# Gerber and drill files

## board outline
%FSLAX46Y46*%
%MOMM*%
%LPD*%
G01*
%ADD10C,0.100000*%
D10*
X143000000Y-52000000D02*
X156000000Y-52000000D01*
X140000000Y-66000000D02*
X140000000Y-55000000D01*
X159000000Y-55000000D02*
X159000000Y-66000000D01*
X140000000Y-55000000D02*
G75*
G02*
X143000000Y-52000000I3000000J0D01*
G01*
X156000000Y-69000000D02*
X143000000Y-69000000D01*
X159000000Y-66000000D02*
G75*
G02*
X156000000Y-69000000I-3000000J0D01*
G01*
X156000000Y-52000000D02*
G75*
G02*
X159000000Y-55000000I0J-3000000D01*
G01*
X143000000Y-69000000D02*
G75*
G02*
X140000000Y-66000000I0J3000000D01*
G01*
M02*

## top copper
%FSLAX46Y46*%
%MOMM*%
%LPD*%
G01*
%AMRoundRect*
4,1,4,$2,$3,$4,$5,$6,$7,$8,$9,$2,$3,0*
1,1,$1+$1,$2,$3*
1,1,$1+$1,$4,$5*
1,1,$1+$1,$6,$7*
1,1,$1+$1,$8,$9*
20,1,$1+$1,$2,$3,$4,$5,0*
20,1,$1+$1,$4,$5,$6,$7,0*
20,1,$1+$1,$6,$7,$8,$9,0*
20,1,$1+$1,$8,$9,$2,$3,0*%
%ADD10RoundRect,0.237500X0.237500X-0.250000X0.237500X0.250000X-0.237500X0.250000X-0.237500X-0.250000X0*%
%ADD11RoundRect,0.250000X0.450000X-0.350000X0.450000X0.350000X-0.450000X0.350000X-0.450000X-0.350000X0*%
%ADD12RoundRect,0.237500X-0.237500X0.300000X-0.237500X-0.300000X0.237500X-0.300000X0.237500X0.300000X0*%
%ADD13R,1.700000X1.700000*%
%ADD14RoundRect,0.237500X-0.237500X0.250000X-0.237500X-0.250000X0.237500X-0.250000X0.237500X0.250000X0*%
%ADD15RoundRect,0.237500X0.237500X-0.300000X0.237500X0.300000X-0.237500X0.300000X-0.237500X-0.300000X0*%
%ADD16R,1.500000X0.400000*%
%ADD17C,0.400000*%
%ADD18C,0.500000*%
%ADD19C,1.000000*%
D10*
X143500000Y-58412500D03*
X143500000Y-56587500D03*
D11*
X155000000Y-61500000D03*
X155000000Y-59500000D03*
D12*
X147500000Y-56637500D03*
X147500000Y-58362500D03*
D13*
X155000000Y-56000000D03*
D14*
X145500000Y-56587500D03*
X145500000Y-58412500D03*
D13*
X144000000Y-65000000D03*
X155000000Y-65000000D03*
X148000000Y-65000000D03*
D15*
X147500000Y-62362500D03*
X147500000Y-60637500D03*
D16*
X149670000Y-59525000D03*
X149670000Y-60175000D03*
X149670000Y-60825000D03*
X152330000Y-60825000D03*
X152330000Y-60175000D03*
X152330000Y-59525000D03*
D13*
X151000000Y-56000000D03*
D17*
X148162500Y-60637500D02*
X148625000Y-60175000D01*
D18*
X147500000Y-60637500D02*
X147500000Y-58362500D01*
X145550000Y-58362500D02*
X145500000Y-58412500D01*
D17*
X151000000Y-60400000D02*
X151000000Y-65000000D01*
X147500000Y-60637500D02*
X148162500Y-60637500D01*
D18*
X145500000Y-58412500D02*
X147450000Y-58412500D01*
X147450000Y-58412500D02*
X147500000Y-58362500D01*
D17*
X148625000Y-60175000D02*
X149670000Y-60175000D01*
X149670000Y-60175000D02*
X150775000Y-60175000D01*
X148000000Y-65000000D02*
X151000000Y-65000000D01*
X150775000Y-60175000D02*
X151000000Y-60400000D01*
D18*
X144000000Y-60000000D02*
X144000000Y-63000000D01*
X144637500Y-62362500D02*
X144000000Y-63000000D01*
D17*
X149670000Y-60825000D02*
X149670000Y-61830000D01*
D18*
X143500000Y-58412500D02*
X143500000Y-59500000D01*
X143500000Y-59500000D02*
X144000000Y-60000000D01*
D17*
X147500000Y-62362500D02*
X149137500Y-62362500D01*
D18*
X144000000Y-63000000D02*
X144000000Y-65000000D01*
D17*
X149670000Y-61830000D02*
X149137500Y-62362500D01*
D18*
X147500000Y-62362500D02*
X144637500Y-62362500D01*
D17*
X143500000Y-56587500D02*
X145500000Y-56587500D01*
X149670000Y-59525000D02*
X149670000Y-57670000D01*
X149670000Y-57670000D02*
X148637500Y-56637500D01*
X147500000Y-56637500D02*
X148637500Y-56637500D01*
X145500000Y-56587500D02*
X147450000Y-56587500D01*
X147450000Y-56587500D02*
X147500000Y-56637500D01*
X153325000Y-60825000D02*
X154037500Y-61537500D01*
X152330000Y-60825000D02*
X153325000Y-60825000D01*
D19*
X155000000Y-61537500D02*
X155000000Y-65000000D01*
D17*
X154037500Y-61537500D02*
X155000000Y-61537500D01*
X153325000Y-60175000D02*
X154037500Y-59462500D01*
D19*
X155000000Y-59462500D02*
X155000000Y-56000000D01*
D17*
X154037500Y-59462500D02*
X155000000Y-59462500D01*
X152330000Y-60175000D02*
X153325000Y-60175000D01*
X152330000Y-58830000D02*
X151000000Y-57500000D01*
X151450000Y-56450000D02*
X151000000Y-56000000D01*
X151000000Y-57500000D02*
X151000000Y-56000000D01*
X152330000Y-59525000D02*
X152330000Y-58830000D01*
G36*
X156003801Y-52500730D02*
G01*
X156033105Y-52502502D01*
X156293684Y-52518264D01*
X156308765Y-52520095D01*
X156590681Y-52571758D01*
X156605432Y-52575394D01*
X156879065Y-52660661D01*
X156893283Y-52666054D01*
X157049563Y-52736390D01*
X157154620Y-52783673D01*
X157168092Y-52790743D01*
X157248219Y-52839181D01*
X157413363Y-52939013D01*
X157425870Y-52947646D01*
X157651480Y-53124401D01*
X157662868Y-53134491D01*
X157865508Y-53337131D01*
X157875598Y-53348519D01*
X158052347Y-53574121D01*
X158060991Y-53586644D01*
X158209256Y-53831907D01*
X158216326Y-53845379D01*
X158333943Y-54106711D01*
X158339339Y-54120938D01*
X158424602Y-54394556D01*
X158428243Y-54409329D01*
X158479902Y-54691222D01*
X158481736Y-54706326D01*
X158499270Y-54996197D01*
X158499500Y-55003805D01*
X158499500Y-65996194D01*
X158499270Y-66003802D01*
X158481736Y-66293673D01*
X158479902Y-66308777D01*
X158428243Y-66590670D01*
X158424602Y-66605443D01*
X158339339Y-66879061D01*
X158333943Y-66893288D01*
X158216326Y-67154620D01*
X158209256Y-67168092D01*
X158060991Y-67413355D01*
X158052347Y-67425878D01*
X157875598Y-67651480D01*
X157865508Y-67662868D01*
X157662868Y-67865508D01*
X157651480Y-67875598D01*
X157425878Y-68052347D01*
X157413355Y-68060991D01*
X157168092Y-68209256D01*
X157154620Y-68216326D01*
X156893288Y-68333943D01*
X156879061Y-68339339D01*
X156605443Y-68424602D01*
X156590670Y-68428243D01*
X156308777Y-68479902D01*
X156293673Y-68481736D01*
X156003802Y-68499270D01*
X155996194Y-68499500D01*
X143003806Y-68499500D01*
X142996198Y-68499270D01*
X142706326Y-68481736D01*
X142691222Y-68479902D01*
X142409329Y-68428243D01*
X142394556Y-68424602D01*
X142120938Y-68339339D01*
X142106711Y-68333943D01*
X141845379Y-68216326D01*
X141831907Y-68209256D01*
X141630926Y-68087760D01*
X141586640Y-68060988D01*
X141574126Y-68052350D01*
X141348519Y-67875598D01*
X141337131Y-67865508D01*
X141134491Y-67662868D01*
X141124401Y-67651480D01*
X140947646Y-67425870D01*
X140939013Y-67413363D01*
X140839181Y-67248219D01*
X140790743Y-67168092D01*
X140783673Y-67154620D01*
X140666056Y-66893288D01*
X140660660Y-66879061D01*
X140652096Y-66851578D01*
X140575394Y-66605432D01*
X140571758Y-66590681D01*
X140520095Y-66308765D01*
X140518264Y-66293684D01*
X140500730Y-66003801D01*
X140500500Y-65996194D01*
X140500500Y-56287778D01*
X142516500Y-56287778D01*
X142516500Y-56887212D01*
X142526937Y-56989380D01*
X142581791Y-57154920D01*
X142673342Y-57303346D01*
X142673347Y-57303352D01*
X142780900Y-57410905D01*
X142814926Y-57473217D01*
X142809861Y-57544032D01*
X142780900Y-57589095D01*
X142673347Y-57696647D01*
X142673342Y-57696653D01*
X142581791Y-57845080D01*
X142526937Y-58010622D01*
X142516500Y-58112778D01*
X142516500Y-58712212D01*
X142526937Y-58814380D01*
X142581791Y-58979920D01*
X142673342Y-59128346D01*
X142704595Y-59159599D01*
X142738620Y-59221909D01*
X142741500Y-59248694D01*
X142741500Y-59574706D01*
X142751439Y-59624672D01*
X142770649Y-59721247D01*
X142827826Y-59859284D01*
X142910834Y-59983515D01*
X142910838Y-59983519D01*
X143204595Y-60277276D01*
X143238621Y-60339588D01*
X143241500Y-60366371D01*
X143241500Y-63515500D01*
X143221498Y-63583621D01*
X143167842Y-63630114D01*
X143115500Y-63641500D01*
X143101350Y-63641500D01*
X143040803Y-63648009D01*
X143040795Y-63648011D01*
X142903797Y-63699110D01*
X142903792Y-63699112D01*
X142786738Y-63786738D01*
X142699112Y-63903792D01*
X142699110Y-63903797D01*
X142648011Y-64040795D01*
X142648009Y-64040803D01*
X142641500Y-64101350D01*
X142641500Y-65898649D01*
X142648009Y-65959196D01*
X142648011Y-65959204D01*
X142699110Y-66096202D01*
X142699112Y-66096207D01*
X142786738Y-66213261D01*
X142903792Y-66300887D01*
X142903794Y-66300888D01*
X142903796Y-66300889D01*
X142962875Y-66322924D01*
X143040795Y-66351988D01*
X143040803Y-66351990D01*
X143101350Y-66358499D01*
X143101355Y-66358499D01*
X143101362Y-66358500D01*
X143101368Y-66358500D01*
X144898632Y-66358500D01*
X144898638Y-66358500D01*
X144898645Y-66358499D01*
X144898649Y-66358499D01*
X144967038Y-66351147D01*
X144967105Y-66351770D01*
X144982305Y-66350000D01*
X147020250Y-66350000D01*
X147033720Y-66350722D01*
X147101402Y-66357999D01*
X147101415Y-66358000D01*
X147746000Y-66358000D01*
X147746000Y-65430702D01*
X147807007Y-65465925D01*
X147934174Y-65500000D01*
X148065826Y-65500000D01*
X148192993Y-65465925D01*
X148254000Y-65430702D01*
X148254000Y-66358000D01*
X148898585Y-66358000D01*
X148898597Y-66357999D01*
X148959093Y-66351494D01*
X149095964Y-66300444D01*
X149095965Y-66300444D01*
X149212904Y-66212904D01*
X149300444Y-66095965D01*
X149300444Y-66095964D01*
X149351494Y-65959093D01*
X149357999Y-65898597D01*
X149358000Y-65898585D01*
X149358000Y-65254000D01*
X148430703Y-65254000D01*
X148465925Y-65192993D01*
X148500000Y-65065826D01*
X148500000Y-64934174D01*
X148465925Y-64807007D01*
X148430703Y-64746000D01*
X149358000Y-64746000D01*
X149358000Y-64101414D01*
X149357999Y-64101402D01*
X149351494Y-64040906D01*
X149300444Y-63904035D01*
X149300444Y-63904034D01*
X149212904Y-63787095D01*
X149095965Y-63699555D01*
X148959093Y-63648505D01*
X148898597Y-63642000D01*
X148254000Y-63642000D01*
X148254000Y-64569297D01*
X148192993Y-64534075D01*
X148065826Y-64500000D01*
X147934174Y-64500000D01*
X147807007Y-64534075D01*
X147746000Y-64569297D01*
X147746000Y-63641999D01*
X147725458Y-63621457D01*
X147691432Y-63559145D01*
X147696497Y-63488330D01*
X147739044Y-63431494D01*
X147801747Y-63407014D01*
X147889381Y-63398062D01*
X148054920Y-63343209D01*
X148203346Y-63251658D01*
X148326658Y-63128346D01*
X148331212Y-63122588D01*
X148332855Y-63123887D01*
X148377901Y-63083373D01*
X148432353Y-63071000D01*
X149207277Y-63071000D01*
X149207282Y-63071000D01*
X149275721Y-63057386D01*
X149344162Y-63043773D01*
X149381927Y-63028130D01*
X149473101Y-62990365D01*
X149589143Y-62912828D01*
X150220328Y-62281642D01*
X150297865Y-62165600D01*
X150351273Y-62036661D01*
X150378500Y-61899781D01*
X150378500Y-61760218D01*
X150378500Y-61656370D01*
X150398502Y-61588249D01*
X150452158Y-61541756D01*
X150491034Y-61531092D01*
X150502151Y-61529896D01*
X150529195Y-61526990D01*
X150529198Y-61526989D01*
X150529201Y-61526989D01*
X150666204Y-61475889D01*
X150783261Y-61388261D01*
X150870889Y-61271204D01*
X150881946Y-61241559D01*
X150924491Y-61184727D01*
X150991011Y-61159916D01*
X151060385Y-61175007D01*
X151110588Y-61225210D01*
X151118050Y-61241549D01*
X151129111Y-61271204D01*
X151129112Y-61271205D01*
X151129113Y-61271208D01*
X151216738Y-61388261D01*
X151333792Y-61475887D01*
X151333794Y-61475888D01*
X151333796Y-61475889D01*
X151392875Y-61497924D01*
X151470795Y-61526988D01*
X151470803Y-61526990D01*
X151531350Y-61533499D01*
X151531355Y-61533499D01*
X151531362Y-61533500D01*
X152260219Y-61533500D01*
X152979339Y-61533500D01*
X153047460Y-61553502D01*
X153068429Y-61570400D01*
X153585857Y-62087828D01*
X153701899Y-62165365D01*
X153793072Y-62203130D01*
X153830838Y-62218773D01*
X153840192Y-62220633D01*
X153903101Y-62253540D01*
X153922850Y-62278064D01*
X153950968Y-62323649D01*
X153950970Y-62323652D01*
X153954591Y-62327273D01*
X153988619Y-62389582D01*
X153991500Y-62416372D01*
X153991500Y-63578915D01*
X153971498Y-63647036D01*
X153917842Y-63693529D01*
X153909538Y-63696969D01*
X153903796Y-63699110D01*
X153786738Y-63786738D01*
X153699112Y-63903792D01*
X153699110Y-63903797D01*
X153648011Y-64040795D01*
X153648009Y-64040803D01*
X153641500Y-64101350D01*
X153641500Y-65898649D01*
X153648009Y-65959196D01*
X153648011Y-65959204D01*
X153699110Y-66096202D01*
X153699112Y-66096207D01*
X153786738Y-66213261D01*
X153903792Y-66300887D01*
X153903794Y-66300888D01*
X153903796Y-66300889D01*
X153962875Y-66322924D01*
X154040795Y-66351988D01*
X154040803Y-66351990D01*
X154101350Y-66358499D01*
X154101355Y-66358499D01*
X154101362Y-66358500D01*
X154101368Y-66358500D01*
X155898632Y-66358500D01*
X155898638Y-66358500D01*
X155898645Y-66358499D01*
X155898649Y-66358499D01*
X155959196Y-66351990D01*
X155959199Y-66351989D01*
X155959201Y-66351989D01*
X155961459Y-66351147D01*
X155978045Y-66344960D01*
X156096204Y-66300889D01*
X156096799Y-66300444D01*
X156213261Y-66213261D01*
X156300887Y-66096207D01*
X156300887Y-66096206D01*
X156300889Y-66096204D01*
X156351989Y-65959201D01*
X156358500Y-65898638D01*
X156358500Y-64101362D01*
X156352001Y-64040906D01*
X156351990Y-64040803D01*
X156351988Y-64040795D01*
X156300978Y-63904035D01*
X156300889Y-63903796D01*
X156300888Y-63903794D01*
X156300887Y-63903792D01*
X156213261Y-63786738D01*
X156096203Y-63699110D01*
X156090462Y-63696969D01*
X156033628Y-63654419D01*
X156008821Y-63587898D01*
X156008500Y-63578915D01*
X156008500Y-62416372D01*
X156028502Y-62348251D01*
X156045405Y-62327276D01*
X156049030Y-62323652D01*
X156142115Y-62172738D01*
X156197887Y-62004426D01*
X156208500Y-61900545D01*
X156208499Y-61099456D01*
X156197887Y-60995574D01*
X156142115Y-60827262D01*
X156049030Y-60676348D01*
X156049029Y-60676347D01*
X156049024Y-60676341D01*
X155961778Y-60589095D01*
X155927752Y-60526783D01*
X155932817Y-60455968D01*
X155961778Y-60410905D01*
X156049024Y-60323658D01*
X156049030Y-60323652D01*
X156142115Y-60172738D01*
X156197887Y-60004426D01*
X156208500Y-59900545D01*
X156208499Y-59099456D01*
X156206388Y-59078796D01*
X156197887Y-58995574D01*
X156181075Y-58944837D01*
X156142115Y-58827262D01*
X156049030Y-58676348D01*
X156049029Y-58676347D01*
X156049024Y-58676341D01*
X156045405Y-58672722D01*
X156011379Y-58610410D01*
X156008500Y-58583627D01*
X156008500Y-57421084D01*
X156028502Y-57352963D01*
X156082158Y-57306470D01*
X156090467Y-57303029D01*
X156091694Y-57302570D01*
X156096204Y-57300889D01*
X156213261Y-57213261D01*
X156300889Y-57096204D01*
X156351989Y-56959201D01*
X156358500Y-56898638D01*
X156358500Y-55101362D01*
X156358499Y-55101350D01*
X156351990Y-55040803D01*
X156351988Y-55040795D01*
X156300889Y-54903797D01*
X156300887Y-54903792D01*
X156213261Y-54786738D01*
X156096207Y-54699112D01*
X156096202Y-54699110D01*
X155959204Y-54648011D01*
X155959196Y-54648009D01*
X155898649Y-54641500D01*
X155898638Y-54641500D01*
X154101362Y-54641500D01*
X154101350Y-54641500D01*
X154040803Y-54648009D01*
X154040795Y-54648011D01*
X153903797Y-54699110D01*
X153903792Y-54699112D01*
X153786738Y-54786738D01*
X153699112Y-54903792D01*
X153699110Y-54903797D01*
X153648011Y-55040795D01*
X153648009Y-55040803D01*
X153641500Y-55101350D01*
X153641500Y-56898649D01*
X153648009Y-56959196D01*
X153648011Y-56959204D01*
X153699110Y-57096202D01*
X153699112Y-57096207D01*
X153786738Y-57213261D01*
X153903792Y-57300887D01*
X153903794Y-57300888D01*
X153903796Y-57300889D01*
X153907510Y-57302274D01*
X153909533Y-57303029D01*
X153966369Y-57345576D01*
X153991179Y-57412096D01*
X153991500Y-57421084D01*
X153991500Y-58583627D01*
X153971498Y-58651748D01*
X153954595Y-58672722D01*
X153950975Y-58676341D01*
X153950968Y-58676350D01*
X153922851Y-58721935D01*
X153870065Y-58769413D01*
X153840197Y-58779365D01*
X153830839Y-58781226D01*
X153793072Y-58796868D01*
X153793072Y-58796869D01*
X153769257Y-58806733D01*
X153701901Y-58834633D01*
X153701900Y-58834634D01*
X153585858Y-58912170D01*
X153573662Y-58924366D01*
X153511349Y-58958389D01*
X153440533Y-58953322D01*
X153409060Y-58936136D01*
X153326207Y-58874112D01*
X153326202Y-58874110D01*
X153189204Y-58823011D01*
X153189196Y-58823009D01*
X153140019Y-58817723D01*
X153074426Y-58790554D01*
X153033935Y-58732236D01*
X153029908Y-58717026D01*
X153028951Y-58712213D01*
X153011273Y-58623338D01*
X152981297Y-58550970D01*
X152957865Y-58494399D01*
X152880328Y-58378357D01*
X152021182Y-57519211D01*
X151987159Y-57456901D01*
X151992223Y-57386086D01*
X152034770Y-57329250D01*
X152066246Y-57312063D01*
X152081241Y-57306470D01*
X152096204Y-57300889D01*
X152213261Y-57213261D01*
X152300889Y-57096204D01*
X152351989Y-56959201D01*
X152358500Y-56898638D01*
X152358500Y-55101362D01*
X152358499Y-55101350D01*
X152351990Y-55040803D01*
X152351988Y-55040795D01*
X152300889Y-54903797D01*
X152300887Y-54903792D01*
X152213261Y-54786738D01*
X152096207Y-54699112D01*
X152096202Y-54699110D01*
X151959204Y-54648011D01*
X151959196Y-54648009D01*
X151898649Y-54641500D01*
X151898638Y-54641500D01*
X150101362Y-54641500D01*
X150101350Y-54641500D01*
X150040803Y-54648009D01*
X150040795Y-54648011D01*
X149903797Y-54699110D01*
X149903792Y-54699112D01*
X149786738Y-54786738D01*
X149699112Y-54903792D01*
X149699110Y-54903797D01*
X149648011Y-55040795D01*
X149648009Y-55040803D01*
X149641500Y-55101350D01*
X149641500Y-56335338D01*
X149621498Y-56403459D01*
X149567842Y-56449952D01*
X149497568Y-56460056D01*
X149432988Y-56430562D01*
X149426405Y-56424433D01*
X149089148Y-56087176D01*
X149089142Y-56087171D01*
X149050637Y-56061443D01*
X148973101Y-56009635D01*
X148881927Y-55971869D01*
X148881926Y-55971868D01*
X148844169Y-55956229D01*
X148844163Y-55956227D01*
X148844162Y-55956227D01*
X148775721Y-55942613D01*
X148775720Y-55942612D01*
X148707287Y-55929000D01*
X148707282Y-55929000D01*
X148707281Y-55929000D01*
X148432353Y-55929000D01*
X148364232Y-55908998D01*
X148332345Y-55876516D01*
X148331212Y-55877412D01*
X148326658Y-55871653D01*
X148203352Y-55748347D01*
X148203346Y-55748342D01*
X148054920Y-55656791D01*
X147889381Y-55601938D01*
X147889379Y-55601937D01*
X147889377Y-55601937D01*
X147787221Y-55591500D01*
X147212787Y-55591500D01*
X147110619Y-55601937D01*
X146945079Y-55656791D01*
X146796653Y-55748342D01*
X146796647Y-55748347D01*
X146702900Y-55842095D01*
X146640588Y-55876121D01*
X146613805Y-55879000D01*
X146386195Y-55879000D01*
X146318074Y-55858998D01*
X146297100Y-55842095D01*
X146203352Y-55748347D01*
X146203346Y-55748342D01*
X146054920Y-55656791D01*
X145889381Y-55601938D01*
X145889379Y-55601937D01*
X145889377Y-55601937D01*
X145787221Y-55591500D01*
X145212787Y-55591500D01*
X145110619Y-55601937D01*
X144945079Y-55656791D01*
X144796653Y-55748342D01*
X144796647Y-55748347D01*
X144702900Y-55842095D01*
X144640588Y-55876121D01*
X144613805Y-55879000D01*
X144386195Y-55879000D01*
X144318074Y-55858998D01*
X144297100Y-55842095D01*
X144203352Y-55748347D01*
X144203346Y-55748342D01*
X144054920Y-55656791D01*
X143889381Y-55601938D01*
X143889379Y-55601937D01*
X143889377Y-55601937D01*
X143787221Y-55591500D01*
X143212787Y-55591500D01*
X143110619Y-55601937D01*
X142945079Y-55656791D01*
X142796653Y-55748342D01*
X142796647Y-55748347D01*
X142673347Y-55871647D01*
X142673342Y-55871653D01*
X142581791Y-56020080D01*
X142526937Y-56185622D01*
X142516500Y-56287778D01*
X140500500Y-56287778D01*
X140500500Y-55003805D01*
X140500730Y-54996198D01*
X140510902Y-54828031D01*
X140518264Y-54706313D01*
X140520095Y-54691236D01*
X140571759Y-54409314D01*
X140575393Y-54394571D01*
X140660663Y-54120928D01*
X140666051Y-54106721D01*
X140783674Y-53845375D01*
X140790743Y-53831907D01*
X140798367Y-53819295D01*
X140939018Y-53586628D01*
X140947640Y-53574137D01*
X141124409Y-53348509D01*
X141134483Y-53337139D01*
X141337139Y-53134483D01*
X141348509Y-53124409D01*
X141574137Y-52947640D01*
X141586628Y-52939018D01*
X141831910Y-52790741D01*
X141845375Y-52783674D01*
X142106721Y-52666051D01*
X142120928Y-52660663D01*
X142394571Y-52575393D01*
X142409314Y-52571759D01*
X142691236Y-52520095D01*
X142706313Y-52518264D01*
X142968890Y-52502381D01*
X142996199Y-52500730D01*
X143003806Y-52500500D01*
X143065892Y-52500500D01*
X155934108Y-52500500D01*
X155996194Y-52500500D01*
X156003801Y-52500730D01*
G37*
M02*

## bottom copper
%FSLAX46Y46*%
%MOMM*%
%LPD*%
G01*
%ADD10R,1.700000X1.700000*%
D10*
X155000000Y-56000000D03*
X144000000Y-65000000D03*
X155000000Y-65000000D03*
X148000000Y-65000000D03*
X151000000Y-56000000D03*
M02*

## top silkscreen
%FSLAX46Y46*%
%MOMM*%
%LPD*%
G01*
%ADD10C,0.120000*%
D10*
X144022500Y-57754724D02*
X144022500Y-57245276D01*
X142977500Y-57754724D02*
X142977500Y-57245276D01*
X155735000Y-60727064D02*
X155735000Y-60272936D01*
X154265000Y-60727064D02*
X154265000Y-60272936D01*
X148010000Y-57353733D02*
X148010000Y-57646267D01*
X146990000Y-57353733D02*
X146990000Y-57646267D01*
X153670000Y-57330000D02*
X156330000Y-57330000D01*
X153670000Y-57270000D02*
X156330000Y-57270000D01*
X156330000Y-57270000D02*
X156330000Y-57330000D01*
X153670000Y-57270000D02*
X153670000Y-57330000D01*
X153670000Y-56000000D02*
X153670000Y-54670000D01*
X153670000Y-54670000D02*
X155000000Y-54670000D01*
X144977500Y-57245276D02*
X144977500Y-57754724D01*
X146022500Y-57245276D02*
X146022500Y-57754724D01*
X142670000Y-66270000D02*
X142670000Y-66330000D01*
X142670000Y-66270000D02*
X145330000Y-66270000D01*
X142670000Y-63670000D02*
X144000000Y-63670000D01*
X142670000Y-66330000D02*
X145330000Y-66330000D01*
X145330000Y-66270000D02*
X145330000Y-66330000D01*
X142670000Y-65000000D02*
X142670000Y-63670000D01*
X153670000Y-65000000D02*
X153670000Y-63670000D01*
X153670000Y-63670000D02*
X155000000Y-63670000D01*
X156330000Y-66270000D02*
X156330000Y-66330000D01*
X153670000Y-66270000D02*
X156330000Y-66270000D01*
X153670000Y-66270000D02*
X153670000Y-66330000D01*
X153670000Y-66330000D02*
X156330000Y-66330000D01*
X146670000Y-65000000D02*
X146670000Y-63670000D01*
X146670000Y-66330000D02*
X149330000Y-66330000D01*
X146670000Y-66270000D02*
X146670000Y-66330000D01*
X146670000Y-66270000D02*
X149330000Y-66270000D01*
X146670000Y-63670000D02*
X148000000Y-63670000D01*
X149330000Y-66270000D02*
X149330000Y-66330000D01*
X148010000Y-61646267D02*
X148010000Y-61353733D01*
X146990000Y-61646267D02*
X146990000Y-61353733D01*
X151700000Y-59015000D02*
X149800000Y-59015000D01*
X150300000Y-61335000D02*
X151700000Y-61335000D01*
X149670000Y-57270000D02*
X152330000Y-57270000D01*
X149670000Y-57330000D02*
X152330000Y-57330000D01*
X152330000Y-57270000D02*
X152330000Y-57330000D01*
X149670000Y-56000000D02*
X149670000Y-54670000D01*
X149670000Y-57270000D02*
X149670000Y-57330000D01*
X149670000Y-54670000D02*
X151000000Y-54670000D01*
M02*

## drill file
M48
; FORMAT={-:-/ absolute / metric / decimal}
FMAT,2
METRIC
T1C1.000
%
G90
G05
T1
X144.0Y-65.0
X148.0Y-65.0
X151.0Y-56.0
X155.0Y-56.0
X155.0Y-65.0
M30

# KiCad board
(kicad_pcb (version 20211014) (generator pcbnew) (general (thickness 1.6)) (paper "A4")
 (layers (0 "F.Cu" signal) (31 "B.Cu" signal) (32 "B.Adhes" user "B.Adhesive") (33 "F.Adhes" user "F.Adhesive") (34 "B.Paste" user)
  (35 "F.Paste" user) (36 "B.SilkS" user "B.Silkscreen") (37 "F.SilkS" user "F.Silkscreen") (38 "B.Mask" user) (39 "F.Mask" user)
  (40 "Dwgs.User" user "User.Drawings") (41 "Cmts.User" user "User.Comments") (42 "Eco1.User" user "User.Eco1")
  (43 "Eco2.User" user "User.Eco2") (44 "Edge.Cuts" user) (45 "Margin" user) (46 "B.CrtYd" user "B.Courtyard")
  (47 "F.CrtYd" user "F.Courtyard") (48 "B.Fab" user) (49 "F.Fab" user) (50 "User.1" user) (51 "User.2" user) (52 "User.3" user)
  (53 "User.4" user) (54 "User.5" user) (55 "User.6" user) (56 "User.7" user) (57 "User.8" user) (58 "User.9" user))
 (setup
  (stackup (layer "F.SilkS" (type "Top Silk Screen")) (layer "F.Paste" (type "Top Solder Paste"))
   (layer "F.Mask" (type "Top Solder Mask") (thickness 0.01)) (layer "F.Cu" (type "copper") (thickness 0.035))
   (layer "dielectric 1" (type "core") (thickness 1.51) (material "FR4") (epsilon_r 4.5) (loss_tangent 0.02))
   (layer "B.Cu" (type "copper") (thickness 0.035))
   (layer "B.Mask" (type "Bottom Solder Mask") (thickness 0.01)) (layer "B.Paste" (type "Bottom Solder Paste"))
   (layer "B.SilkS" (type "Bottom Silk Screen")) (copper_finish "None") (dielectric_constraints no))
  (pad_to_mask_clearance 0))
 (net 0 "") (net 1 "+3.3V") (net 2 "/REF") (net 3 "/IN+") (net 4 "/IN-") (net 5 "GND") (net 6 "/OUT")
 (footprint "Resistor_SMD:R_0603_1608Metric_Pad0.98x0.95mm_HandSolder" (layer "F.Cu") (at 143.5 57.5 90)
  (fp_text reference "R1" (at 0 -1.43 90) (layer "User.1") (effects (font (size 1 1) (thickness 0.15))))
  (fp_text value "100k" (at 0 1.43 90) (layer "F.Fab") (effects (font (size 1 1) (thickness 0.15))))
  (fp_line (start -0.254724 0.5225) (end 0.254724 0.5225) (layer "F.SilkS") (width 0.12))
  (fp_line (start -0.254724 -0.5225) (end 0.254724 -0.5225) (layer "F.SilkS") (width 0.12))
  (pad "1" smd roundrect (at -0.9125 0 90) (size 0.975 0.95) (layers "F.Cu" "F.Paste" "F.Mask") (roundrect_rratio 0.25) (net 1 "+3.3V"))
  (pad "2" smd roundrect (at 0.9125 0 90) (size 0.975 0.95) (layers "F.Cu" "F.Paste" "F.Mask") (roundrect_rratio 0.25) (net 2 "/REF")))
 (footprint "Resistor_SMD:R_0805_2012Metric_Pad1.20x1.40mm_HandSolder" (layer "F.Cu") (at 155 60.5 90)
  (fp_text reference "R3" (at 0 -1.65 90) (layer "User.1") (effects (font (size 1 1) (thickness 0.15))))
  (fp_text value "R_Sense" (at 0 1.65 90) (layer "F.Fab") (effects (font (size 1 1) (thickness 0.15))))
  (fp_line (start -0.227064 0.735) (end 0.227064 0.735) (layer "F.SilkS") (width 0.12))
  (fp_line (start -0.227064 -0.735) (end 0.227064 -0.735) (layer "F.SilkS") (width 0.12))
  (pad "1" smd roundrect (at -1 0 90) (size 1.2 1.4) (layers "F.Cu" "F.Paste" "F.Mask") (roundrect_rratio 0.208333) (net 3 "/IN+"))
  (pad "2" smd roundrect (at 1 0 90) (size 1.2 1.4) (layers "F.Cu" "F.Paste" "F.Mask") (roundrect_rratio 0.208333) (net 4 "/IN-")))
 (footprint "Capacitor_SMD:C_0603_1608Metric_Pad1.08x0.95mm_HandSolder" (layer "F.Cu") (at 147.5 57.5 -90)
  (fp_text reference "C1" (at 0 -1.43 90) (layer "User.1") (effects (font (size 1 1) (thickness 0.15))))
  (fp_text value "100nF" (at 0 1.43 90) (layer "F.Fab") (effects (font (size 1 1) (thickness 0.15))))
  (fp_line (start -0.146267 -0.51) (end 0.146267 -0.51) (layer "F.SilkS") (width 0.12))
  (fp_line (start -0.146267 0.51) (end 0.146267 0.51) (layer "F.SilkS") (width 0.12))
  (pad "1" smd roundrect (at -0.8625 0 270) (size 1.075 0.95) (layers "F.Cu" "F.Paste" "F.Mask") (roundrect_rratio 0.25) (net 2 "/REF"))
  (pad "2" smd roundrect (at 0.8625 0 270) (size 1.075 0.95) (layers "F.Cu" "F.Paste" "F.Mask") (roundrect_rratio 0.25) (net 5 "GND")))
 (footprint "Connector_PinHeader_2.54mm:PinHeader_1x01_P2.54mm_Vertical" (layer "F.Cu") (at 155 56)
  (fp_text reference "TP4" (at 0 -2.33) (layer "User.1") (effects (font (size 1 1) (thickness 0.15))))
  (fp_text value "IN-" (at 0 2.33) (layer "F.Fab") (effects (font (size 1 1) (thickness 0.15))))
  (fp_line (start -1.33 1.33) (end 1.33 1.33) (layer "F.SilkS") (width 0.12))
  (fp_line (start -1.33 1.27) (end 1.33 1.27) (layer "F.SilkS") (width 0.12))
  (fp_line (start 1.33 1.27) (end 1.33 1.33) (layer "F.SilkS") (width 0.12))
  (fp_line (start -1.33 1.27) (end -1.33 1.33) (layer "F.SilkS") (width 0.12))
  (fp_line (start -1.33 0) (end -1.33 -1.33) (layer "F.SilkS") (width 0.12))
  (fp_line (start -1.33 -1.33) (end 0 -1.33) (layer "F.SilkS") (width 0.12))
  (pad "1" thru_hole rect (at 0 0) (size 1.7 1.7) (drill 1) (layers *.Cu *.Mask) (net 4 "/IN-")))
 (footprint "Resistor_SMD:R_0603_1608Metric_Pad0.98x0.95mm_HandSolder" (layer "F.Cu") (at 145.5 57.5 -90)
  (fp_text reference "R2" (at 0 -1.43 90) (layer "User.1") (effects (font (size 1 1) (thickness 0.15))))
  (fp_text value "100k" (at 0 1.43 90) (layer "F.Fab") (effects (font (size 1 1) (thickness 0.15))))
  (fp_line (start -0.254724 0.5225) (end 0.254724 0.5225) (layer "F.SilkS") (width 0.12))
  (fp_line (start -0.254724 -0.5225) (end 0.254724 -0.5225) (layer "F.SilkS") (width 0.12))
  (pad "1" smd roundrect (at -0.9125 0 270) (size 0.975 0.95) (layers "F.Cu" "F.Paste" "F.Mask") (roundrect_rratio 0.25) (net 2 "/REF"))
  (pad "2" smd roundrect (at 0.9125 0 270) (size 0.975 0.95) (layers "F.Cu" "F.Paste" "F.Mask") (roundrect_rratio 0.25) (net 5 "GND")))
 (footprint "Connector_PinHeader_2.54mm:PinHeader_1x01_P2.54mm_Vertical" (layer "F.Cu") (at 144 65)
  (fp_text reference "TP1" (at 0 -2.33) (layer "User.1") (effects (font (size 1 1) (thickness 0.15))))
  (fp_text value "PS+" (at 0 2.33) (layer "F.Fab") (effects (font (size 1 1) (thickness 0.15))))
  (fp_line (start -1.33 1.27) (end -1.33 1.33) (layer "F.SilkS") (width 0.12))
  (fp_line (start -1.33 1.27) (end 1.33 1.27) (layer "F.SilkS") (width 0.12))
  (fp_line (start -1.33 -1.33) (end 0 -1.33) (layer "F.SilkS") (width 0.12))
  (fp_line (start -1.33 1.33) (end 1.33 1.33) (layer "F.SilkS") (width 0.12))
  (fp_line (start 1.33 1.27) (end 1.33 1.33) (layer "F.SilkS") (width 0.12))
  (fp_line (start -1.33 0) (end -1.33 -1.33) (layer "F.SilkS") (width 0.12))
  (pad "1" thru_hole rect (at 0 0) (size 1.7 1.7) (drill 1) (layers *.Cu *.Mask) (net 1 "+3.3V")))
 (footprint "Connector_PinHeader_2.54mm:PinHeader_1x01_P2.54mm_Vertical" (layer "F.Cu") (at 155 65)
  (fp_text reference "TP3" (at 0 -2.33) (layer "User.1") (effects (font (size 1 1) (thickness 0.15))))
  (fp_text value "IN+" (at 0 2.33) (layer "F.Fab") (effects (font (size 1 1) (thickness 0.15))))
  (fp_line (start -1.33 0) (end -1.33 -1.33) (layer "F.SilkS") (width 0.12))
  (fp_line (start -1.33 -1.33) (end 0 -1.33) (layer "F.SilkS") (width 0.12))
  (fp_line (start 1.33 1.27) (end 1.33 1.33) (layer "F.SilkS") (width 0.12))
  (fp_line (start -1.33 1.27) (end 1.33 1.27) (layer "F.SilkS") (width 0.12))
  (fp_line (start -1.33 1.27) (end -1.33 1.33) (layer "F.SilkS") (width 0.12))
  (fp_line (start -1.33 1.33) (end 1.33 1.33) (layer "F.SilkS") (width 0.12))
  (pad "1" thru_hole rect (at 0 0) (size 1.7 1.7) (drill 1) (layers *.Cu *.Mask) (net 3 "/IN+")))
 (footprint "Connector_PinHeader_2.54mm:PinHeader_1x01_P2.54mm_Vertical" (layer "F.Cu") (at 148 65)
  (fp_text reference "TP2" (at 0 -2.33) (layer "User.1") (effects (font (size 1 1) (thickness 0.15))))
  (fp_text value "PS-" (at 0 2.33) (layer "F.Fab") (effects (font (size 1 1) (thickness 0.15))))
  (fp_line (start -1.33 0) (end -1.33 -1.33) (layer "F.SilkS") (width 0.12))
  (fp_line (start -1.33 1.33) (end 1.33 1.33) (layer "F.SilkS") (width 0.12))
  (fp_line (start -1.33 1.27) (end -1.33 1.33) (layer "F.SilkS") (width 0.12))
  (fp_line (start -1.33 1.27) (end 1.33 1.27) (layer "F.SilkS") (width 0.12))
  (fp_line (start -1.33 -1.33) (end 0 -1.33) (layer "F.SilkS") (width 0.12))
  (fp_line (start 1.33 1.27) (end 1.33 1.33) (layer "F.SilkS") (width 0.12))
  (pad "1" thru_hole rect (at 0 0) (size 1.7 1.7) (drill 1) (layers *.Cu *.Mask) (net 5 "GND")))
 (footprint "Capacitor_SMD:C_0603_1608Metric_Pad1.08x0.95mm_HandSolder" (layer "F.Cu") (at 147.5 61.5 90)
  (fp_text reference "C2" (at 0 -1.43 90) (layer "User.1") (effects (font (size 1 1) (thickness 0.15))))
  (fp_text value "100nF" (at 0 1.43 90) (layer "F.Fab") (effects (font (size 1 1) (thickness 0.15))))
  (fp_line (start -0.146267 0.51) (end 0.146267 0.51) (layer "F.SilkS") (width 0.12))
  (fp_line (start -0.146267 -0.51) (end 0.146267 -0.51) (layer "F.SilkS") (width 0.12))
  (pad "1" smd roundrect (at -0.8625 0 90) (size 1.075 0.95) (layers "F.Cu" "F.Paste" "F.Mask") (roundrect_rratio 0.25) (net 1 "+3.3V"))
  (pad "2" smd roundrect (at 0.8625 0 90) (size 1.075 0.95) (layers "F.Cu" "F.Paste" "F.Mask") (roundrect_rratio 0.25) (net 5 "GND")))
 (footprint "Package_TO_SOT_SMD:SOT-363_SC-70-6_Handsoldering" (layer "F.Cu") (at 151 60.175)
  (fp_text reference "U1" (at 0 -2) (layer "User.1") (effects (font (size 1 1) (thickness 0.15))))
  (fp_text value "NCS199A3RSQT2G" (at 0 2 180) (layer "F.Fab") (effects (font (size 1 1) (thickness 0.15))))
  (fp_line (start 0.7 -1.16) (end -1.2 -1.16) (layer "F.SilkS") (width 0.12))
  (fp_line (start -0.7 1.16) (end 0.7 1.16) (layer "F.SilkS") (width 0.12))
  (pad "1" smd rect (at -1.33 -0.65) (size 1.5 0.4) (layers "F.Cu" "F.Paste" "F.Mask") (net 2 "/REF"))
  (pad "2" smd rect (at -1.33 0) (size 1.5 0.4) (layers "F.Cu" "F.Paste" "F.Mask") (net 5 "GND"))
  (pad "3" smd rect (at -1.33 0.65) (size 1.5 0.4) (layers "F.Cu" "F.Paste" "F.Mask") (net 1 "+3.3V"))
  (pad "4" smd rect (at 1.33 0.65) (size 1.5 0.4) (layers "F.Cu" "F.Paste" "F.Mask") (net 3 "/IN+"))
  (pad "5" smd rect (at 1.33 0) (size 1.5 0.4) (layers "F.Cu" "F.Paste" "F.Mask") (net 4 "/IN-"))
  (pad "6" smd rect (at 1.33 -0.65) (size 1.5 0.4) (layers "F.Cu" "F.Paste" "F.Mask") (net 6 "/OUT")))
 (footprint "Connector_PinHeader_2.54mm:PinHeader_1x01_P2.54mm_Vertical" (layer "F.Cu") (at 151 56)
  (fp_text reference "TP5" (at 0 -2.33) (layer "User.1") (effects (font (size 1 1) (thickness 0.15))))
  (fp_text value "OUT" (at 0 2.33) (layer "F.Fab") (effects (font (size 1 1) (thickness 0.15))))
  (fp_line (start -1.33 1.27) (end 1.33 1.27) (layer "F.SilkS") (width 0.12))
  (fp_line (start -1.33 1.33) (end 1.33 1.33) (layer "F.SilkS") (width 0.12))
  (fp_line (start 1.33 1.27) (end 1.33 1.33) (layer "F.SilkS") (width 0.12))
  (fp_line (start -1.33 0) (end -1.33 -1.33) (layer "F.SilkS") (width 0.12))
  (fp_line (start -1.33 1.27) (end -1.33 1.33) (layer "F.SilkS") (width 0.12))
  (fp_line (start -1.33 -1.33) (end 0 -1.33) (layer "F.SilkS") (width 0.12))
  (pad "1" thru_hole rect (at 0 0) (size 1.7 1.7) (drill 1) (layers *.Cu *.Mask) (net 6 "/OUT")))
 (gr_line (start 143 52) (end 156 52) (layer "Edge.Cuts") (width 0.1))
 (gr_line (start 140 66) (end 140 55) (layer "Edge.Cuts") (width 0.1))
 (gr_line (start 159 55) (end 159 66) (layer "Edge.Cuts") (width 0.1))
 (gr_arc (start 140 55) (mid 140.87868 52.87868) (end 143 52) (layer "Edge.Cuts") (width 0.1))
 (gr_line (start 156 69) (end 143 69) (layer "Edge.Cuts") (width 0.1))
 (gr_arc (start 159 66) (mid 158.12132 68.12132) (end 156 69) (layer "Edge.Cuts") (width 0.1))
 (gr_arc (start 156 52) (mid 158.12132 52.87868) (end 159 55) (layer "Edge.Cuts") (width 0.1))
 (gr_arc (start 143 69) (mid 140.87868 68.12132) (end 140 66) (layer "Edge.Cuts") (width 0.1))
 (segment (start 148.1625 60.6375) (end 148.625 60.175) (width 0.4) (layer "F.Cu") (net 5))
 (segment (start 147.5 60.6375) (end 147.5 58.3625) (width 0.5) (layer "F.Cu") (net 5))
 (segment (start 145.55 58.3625) (end 145.5 58.4125) (width 0.5) (layer "F.Cu") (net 5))
 (segment (start 151 60.4) (end 151 65) (width 0.4) (layer "F.Cu") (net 5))
 (segment (start 147.5 60.6375) (end 148.1625 60.6375) (width 0.4) (layer "F.Cu") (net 5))
 (segment (start 145.5 58.4125) (end 147.45 58.4125) (width 0.5) (layer "F.Cu") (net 5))
 (segment (start 147.45 58.4125) (end 147.5 58.3625) (width 0.5) (layer "F.Cu") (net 5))
 (segment (start 148.625 60.175) (end 149.67 60.175) (width 0.4) (layer "F.Cu") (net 5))
 (segment (start 149.67 60.175) (end 150.775 60.175) (width 0.4) (layer "F.Cu") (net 5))
 (segment (start 148 65) (end 151 65) (width 0.4) (layer "F.Cu") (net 5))
 (segment (start 150.775 60.175) (end 151 60.4) (width 0.4) (layer "F.Cu") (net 5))
 (segment (start 144 60) (end 144 63) (width 0.5) (layer "F.Cu") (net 1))
 (segment (start 144.6375 62.3625) (end 144 63) (width 0.5) (layer "F.Cu") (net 1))
 (segment (start 149.67 60.825) (end 149.67 61.83) (width 0.4) (layer "F.Cu") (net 1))
 (segment (start 143.5 58.4125) (end 143.5 59.5) (width 0.5) (layer "F.Cu") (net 1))
 (segment (start 143.5 59.5) (end 144 60) (width 0.5) (layer "F.Cu") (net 1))
 (segment (start 147.5 62.3625) (end 149.1375 62.3625) (width 0.4) (layer "F.Cu") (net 1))
 (segment (start 144 63) (end 144 65) (width 0.5) (layer "F.Cu") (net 1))
 (segment (start 149.67 61.83) (end 149.1375 62.3625) (width 0.4) (layer "F.Cu") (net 1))
 (segment (start 147.5 62.3625) (end 144.6375 62.3625) (width 0.5) (layer "F.Cu") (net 1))
 (segment (start 143.5 56.5875) (end 145.5 56.5875) (width 0.4) (layer "F.Cu") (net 2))
 (segment (start 149.67 59.525) (end 149.67 57.67) (width 0.4) (layer "F.Cu") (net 2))
 (segment (start 149.67 57.67) (end 148.6375 56.6375) (width 0.4) (layer "F.Cu") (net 2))
 (segment (start 147.5 56.6375) (end 148.6375 56.6375) (width 0.4) (layer "F.Cu") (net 2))
 (segment (start 145.5 56.5875) (end 147.45 56.5875) (width 0.4) (layer "F.Cu") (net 2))
 (segment (start 147.45 56.5875) (end 147.5 56.6375) (width 0.4) (layer "F.Cu") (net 2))
 (segment (start 153.325 60.825) (end 154.0375 61.5375) (width 0.4) (layer "F.Cu") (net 3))
 (segment (start 152.33 60.825) (end 153.325 60.825) (width 0.4) (layer "F.Cu") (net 3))
 (segment (start 155 61.5375) (end 155 65) (width 1) (layer "F.Cu") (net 3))
 (segment (start 154.0375 61.5375) (end 155 61.5375) (width 0.4) (layer "F.Cu") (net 3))
 (segment (start 153.325 60.175) (end 154.0375 59.4625) (width 0.4) (layer "F.Cu") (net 4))
 (segment (start 155 59.4625) (end 155 56) (width 1) (layer "F.Cu") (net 4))
 (segment (start 154.0375 59.4625) (end 155 59.4625) (width 0.4) (layer "F.Cu") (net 4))
 (segment (start 152.33 60.175) (end 153.325 60.175) (width 0.4) (layer "F.Cu") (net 4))
 (segment (start 152.33 58.83) (end 151 57.5) (width 0.4) (layer "F.Cu") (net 6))
 (segment (start 151.45 56.45) (end 151 56) (width 0.4) (layer "F.Cu") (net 6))
 (segment (start 151 57.5) (end 151 56) (width 0.4) (layer "F.Cu") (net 6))
 (segment (start 152.33 59.525) (end 152.33 58.83) (width 0.4) (layer "F.Cu") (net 6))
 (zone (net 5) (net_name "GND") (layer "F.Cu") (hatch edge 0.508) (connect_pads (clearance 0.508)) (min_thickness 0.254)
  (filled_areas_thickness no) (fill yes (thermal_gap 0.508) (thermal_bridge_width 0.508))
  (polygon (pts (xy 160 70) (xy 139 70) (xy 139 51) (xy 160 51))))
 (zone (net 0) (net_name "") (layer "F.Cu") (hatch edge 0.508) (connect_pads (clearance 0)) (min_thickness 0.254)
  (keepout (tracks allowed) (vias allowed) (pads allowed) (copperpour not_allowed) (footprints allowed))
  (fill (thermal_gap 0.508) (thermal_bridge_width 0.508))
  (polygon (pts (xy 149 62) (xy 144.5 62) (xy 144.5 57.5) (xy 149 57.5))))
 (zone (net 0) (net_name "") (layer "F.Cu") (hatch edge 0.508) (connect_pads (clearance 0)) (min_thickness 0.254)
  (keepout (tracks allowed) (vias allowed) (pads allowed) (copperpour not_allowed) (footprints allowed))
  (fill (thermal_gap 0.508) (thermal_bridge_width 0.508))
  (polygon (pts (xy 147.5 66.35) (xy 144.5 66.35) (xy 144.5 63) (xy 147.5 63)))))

